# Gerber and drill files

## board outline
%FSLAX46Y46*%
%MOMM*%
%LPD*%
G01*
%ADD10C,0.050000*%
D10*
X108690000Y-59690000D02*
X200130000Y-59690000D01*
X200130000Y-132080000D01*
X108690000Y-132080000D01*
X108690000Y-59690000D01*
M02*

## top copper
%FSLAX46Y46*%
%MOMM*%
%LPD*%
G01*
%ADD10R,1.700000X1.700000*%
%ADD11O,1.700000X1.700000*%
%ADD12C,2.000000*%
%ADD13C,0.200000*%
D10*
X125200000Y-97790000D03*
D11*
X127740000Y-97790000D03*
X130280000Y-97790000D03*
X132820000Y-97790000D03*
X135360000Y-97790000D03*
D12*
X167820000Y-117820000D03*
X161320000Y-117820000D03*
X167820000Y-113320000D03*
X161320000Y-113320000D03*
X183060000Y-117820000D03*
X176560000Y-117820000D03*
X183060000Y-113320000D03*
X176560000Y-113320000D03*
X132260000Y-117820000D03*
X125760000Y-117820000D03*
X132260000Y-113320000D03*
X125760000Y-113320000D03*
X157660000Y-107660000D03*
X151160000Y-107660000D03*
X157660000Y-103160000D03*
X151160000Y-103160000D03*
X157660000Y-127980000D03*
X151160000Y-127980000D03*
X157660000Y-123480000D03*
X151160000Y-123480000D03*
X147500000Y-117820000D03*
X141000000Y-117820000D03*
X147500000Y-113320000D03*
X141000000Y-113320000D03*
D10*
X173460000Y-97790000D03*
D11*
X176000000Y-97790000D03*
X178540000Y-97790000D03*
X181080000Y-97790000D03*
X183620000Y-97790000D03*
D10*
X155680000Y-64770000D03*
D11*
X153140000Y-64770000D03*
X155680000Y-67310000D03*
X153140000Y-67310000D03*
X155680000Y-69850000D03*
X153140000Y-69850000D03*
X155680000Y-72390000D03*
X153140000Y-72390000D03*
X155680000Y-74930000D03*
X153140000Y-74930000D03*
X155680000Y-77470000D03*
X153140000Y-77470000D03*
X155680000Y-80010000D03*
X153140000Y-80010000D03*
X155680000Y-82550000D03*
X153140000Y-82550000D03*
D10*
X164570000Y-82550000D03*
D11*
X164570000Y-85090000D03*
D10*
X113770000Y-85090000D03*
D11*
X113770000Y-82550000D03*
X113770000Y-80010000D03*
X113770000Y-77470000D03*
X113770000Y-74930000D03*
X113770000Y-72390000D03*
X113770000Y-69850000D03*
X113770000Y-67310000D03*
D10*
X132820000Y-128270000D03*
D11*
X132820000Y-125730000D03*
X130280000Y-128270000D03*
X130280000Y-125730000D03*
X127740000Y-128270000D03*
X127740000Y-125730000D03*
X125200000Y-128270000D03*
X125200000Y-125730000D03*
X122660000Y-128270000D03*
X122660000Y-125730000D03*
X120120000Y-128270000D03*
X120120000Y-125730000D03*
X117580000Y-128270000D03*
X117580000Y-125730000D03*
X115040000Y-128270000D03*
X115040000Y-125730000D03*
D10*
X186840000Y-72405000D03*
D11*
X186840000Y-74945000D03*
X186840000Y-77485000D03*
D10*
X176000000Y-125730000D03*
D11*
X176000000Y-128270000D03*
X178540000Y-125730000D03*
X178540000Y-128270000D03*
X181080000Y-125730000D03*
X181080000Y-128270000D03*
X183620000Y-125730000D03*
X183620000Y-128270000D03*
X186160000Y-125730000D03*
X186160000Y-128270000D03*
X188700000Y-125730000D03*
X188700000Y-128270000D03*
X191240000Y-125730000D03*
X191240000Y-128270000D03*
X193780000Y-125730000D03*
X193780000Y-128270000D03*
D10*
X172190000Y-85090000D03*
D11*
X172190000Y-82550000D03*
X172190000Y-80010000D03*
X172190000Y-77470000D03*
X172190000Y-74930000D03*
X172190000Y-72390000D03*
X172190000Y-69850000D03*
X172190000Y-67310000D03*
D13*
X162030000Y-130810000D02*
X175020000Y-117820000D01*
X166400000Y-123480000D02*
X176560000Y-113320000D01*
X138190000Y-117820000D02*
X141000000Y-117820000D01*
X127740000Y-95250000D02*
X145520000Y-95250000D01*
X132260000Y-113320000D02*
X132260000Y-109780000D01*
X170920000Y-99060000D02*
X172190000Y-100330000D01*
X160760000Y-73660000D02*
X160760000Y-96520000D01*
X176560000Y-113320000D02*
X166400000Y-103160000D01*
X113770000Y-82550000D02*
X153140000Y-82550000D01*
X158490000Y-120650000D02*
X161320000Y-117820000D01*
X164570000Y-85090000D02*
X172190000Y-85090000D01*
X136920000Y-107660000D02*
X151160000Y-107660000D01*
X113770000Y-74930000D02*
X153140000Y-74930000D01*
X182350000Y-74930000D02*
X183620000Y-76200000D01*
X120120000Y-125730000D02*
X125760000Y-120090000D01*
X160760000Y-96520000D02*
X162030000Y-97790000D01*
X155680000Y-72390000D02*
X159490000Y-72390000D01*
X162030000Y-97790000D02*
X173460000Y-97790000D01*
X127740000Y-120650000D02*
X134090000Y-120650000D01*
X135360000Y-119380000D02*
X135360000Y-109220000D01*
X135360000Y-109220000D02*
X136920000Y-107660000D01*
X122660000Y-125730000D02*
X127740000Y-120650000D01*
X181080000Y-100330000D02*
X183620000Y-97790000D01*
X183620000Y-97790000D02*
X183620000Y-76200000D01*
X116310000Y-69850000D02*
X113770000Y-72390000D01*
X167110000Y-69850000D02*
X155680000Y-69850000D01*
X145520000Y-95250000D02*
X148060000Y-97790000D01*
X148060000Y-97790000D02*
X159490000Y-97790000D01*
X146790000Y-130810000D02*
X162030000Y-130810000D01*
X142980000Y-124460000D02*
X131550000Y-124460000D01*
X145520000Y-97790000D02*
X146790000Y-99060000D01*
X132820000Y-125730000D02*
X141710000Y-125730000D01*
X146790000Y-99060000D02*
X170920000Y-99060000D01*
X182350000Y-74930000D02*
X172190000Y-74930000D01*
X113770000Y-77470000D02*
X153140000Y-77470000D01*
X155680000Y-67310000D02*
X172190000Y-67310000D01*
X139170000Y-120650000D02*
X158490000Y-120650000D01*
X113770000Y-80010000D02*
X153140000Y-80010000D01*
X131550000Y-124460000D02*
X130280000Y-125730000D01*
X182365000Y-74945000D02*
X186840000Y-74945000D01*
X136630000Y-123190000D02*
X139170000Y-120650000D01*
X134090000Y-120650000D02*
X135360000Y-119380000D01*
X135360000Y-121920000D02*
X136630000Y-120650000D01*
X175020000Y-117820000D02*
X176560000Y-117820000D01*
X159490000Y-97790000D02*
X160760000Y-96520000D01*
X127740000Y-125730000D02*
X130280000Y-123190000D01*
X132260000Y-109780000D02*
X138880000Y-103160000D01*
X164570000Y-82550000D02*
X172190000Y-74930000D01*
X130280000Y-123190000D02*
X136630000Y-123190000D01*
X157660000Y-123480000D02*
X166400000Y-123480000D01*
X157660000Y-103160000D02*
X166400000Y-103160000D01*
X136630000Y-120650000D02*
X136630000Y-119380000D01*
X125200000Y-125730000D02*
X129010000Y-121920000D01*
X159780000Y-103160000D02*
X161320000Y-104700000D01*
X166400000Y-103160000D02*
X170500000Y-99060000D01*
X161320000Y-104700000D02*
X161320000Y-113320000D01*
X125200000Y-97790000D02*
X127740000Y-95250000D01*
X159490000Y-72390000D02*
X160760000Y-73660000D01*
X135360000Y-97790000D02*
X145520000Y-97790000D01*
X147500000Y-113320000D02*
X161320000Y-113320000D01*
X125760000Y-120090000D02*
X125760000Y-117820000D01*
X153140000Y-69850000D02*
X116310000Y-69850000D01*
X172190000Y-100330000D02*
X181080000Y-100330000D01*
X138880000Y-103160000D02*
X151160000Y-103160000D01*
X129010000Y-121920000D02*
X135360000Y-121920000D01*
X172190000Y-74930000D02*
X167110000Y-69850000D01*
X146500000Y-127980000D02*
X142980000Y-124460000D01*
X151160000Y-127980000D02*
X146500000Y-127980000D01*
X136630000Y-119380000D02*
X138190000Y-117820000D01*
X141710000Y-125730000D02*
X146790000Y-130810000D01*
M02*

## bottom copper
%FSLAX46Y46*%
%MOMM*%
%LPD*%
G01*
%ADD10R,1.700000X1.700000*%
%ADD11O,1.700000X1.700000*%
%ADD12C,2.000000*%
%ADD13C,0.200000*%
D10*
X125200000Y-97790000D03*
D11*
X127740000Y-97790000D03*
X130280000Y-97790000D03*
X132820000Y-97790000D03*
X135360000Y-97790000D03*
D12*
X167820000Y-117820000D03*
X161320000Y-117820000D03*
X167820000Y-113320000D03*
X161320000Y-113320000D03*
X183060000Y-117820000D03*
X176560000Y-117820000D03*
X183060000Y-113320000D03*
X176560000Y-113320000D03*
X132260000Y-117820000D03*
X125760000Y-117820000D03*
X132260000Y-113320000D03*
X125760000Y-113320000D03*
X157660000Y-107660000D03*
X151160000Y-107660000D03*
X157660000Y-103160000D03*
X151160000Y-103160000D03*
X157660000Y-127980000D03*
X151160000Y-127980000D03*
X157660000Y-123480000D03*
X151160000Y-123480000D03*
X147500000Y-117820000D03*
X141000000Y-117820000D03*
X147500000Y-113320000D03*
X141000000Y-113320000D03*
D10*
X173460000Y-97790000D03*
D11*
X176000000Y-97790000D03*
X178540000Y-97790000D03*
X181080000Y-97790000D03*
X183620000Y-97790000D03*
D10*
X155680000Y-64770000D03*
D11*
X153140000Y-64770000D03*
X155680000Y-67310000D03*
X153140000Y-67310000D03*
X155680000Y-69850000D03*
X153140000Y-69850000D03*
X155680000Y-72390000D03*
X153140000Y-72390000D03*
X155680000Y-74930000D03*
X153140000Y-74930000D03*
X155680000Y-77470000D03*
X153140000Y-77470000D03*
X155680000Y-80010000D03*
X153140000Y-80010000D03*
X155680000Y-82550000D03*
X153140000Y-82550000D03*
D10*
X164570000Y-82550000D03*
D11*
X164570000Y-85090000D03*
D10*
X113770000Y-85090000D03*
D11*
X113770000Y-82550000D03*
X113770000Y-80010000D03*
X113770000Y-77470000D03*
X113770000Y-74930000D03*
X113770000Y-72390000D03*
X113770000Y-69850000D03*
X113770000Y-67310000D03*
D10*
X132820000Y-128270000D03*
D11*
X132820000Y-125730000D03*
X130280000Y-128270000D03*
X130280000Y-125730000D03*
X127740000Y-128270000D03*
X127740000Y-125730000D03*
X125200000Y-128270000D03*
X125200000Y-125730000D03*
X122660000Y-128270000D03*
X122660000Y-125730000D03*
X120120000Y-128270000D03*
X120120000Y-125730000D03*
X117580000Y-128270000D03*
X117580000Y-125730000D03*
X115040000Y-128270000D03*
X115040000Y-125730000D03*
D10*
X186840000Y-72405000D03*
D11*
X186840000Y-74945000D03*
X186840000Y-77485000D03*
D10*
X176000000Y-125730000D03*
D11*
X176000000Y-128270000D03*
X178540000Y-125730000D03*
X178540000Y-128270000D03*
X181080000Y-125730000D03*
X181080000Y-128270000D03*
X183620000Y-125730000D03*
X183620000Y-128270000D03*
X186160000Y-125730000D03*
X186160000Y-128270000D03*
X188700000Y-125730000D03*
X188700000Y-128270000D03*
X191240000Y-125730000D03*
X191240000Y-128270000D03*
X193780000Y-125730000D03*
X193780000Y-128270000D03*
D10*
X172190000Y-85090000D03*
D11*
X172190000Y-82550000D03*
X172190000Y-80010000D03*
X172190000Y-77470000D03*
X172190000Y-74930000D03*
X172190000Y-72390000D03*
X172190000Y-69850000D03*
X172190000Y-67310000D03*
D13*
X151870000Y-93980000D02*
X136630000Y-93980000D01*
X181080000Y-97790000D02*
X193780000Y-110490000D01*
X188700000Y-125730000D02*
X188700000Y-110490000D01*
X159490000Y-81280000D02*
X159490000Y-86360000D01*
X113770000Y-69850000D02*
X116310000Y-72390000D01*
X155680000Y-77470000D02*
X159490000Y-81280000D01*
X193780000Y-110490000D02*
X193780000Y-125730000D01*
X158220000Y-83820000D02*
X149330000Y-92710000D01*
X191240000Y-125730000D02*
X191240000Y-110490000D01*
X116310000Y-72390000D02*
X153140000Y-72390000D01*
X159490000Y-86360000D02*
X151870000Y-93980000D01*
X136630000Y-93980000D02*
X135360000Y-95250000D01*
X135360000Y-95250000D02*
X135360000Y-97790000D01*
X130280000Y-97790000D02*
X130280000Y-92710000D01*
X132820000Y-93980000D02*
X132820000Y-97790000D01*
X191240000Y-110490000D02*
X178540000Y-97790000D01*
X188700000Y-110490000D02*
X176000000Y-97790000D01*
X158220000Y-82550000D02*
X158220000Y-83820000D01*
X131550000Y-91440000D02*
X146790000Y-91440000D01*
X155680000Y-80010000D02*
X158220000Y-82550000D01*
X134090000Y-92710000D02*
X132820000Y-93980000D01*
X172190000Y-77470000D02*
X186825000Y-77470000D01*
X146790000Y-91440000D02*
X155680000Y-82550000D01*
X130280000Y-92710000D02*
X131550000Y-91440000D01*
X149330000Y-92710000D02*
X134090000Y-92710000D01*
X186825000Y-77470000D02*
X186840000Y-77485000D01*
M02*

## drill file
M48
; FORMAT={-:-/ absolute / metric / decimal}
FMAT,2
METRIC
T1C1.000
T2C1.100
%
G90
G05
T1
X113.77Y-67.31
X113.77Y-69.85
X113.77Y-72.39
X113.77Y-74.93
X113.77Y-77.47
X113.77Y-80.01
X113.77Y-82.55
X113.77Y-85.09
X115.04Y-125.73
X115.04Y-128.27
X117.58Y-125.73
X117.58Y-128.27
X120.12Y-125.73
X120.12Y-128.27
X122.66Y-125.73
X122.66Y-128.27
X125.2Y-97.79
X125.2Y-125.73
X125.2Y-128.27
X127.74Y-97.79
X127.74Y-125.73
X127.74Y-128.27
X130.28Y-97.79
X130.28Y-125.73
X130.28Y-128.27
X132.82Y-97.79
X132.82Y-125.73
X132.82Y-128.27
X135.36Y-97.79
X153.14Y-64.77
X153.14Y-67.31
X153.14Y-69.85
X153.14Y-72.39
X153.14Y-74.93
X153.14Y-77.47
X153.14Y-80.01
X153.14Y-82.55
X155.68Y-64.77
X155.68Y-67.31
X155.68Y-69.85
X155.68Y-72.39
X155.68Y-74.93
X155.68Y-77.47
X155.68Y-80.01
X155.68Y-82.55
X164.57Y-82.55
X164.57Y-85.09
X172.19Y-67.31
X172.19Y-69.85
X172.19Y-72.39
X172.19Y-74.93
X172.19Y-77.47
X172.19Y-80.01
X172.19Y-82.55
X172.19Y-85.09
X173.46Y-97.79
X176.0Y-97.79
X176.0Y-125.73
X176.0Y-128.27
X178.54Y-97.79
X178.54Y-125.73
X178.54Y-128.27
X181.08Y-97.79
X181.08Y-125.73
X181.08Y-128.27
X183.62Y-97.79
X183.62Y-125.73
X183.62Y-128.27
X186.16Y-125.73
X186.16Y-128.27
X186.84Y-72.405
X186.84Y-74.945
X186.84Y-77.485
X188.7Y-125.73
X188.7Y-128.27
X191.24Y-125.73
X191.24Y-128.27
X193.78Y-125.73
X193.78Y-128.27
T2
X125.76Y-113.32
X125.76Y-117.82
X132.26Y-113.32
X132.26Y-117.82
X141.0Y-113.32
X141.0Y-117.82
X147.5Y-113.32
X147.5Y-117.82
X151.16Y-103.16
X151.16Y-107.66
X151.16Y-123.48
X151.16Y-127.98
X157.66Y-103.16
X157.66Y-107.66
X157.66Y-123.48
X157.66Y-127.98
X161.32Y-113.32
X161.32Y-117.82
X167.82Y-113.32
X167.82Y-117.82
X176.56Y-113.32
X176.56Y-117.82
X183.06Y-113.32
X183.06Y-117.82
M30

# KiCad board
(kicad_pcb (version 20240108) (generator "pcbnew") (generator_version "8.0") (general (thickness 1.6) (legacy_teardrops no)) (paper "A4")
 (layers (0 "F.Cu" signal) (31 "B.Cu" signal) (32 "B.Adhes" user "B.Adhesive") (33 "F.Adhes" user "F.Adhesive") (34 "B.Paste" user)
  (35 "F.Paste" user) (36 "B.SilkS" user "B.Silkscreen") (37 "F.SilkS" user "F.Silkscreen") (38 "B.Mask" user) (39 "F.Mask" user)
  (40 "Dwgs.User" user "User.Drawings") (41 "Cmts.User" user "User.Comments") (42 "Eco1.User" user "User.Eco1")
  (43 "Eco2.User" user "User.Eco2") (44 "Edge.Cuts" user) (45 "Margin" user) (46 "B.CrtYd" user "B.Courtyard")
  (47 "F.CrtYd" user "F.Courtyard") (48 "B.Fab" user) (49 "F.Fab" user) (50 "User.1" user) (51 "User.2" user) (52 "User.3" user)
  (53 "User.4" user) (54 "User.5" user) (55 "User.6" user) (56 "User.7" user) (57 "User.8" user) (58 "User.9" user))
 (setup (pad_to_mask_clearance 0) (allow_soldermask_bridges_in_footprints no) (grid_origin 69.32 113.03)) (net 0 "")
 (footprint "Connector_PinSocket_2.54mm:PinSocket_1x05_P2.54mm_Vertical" (layer "F.Cu") (at 125.2 97.79 90)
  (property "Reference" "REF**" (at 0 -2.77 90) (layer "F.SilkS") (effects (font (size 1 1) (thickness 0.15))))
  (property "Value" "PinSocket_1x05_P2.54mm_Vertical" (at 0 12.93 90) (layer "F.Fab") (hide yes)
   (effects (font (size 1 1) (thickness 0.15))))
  (pad "1" thru_hole rect (at 0 0 90) (size 1.7 1.7) (drill 1) (layers "*.Cu" "*.Mask") (remove_unused_layers no))
  (pad "2" thru_hole oval (at 0 2.54 90) (size 1.7 1.7) (drill 1) (layers "*.Cu" "*.Mask") (remove_unused_layers no))
  (pad "3" thru_hole oval (at 0 5.08 90) (size 1.7 1.7) (drill 1) (layers "*.Cu" "*.Mask") (remove_unused_layers no))
  (pad "4" thru_hole oval (at 0 7.62 90) (size 1.7 1.7) (drill 1) (layers "*.Cu" "*.Mask") (remove_unused_layers no))
  (pad "5" thru_hole oval (at 0 10.16 90) (size 1.7 1.7) (drill 1) (layers "*.Cu" "*.Mask") (remove_unused_layers no)))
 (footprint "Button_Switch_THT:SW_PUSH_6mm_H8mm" (layer "F.Cu") (at 167.82 117.82 180)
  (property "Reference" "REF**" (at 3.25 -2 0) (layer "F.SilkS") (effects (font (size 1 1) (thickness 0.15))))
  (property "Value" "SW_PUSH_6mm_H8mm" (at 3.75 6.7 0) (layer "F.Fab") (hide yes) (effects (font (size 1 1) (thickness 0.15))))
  (pad "1" thru_hole circle (at 0 0 270) (size 2 2) (drill 1.1) (layers "*.Cu" "*.Mask") (remove_unused_layers no))
  (pad "1" thru_hole circle (at 6.5 0 270) (size 2 2) (drill 1.1) (layers "*.Cu" "*.Mask") (remove_unused_layers no))
  (pad "2" thru_hole circle (at 0 4.5 270) (size 2 2) (drill 1.1) (layers "*.Cu" "*.Mask") (remove_unused_layers no))
  (pad "2" thru_hole circle (at 6.5 4.5 270) (size 2 2) (drill 1.1) (layers "*.Cu" "*.Mask") (remove_unused_layers no)))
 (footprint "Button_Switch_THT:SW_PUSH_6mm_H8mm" (layer "F.Cu") (at 183.06 117.82 180)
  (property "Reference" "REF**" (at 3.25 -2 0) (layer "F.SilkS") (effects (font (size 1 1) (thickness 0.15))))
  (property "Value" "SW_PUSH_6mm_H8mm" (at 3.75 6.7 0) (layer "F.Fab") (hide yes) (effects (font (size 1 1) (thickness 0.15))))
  (pad "1" thru_hole circle (at 0 0 270) (size 2 2) (drill 1.1) (layers "*.Cu" "*.Mask") (remove_unused_layers no))
  (pad "1" thru_hole circle (at 6.5 0 270) (size 2 2) (drill 1.1) (layers "*.Cu" "*.Mask") (remove_unused_layers no))
  (pad "2" thru_hole circle (at 0 4.5 270) (size 2 2) (drill 1.1) (layers "*.Cu" "*.Mask") (remove_unused_layers no))
  (pad "2" thru_hole circle (at 6.5 4.5 270) (size 2 2) (drill 1.1) (layers "*.Cu" "*.Mask") (remove_unused_layers no)))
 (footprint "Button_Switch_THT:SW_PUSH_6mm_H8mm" (layer "F.Cu") (at 132.26 117.82 180)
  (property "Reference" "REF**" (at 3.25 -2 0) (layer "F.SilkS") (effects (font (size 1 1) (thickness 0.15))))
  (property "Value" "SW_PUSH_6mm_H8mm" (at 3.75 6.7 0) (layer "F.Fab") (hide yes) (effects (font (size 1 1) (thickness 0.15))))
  (pad "1" thru_hole circle (at 0 0 270) (size 2 2) (drill 1.1) (layers "*.Cu" "*.Mask") (remove_unused_layers no))
  (pad "1" thru_hole circle (at 6.5 0 270) (size 2 2) (drill 1.1) (layers "*.Cu" "*.Mask") (remove_unused_layers no))
  (pad "2" thru_hole circle (at 0 4.5 270) (size 2 2) (drill 1.1) (layers "*.Cu" "*.Mask") (remove_unused_layers no))
  (pad "2" thru_hole circle (at 6.5 4.5 270) (size 2 2) (drill 1.1) (layers "*.Cu" "*.Mask") (remove_unused_layers no)))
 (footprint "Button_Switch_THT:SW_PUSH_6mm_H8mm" (layer "F.Cu") (at 157.66 107.66 180)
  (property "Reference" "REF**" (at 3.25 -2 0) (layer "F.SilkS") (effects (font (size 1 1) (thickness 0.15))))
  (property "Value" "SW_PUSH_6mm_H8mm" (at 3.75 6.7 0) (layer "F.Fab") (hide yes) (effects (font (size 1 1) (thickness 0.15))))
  (pad "1" thru_hole circle (at 0 0 270) (size 2 2) (drill 1.1) (layers "*.Cu" "*.Mask") (remove_unused_layers no))
  (pad "1" thru_hole circle (at 6.5 0 270) (size 2 2) (drill 1.1) (layers "*.Cu" "*.Mask") (remove_unused_layers no))
  (pad "2" thru_hole circle (at 0 4.5 270) (size 2 2) (drill 1.1) (layers "*.Cu" "*.Mask") (remove_unused_layers no))
  (pad "2" thru_hole circle (at 6.5 4.5 270) (size 2 2) (drill 1.1) (layers "*.Cu" "*.Mask") (remove_unused_layers no)))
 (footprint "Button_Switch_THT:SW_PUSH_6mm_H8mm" (layer "F.Cu") (at 157.66 127.98 180)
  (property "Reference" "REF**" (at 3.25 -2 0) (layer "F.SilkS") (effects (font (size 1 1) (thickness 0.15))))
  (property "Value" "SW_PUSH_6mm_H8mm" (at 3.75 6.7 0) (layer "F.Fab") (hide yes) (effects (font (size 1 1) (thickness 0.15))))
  (pad "1" thru_hole circle (at 0 0 270) (size 2 2) (drill 1.1) (layers "*.Cu" "*.Mask") (remove_unused_layers no))
  (pad "1" thru_hole circle (at 6.5 0 270) (size 2 2) (drill 1.1) (layers "*.Cu" "*.Mask") (remove_unused_layers no))
  (pad "2" thru_hole circle (at 0 4.5 270) (size 2 2) (drill 1.1) (layers "*.Cu" "*.Mask") (remove_unused_layers no))
  (pad "2" thru_hole circle (at 6.5 4.5 270) (size 2 2) (drill 1.1) (layers "*.Cu" "*.Mask") (remove_unused_layers no)))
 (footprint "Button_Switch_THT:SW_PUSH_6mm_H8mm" (layer "F.Cu") (at 147.5 117.82 180)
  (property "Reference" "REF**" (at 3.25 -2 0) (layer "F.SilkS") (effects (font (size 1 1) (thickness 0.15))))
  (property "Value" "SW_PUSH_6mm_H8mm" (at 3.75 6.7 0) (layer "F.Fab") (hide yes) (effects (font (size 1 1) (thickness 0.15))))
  (pad "1" thru_hole circle (at 0 0 270) (size 2 2) (drill 1.1) (layers "*.Cu" "*.Mask") (remove_unused_layers no))
  (pad "1" thru_hole circle (at 6.5 0 270) (size 2 2) (drill 1.1) (layers "*.Cu" "*.Mask") (remove_unused_layers no))
  (pad "2" thru_hole circle (at 0 4.5 270) (size 2 2) (drill 1.1) (layers "*.Cu" "*.Mask") (remove_unused_layers no))
  (pad "2" thru_hole circle (at 6.5 4.5 270) (size 2 2) (drill 1.1) (layers "*.Cu" "*.Mask") (remove_unused_layers no)))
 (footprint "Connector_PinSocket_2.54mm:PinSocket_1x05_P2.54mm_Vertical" (layer "F.Cu") (at 173.46 97.79 90)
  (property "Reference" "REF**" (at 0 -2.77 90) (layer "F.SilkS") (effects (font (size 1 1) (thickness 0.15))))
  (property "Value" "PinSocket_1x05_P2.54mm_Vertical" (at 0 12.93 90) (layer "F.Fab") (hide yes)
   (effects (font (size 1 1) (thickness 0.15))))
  (pad "1" thru_hole rect (at 0 0 90) (size 1.7 1.7) (drill 1) (layers "*.Cu" "*.Mask") (remove_unused_layers no))
  (pad "2" thru_hole oval (at 0 2.54 90) (size 1.7 1.7) (drill 1) (layers "*.Cu" "*.Mask") (remove_unused_layers no))
  (pad "3" thru_hole oval (at 0 5.08 90) (size 1.7 1.7) (drill 1) (layers "*.Cu" "*.Mask") (remove_unused_layers no))
  (pad "4" thru_hole oval (at 0 7.62 90) (size 1.7 1.7) (drill 1) (layers "*.Cu" "*.Mask") (remove_unused_layers no))
  (pad "5" thru_hole oval (at 0 10.16 90) (size 1.7 1.7) (drill 1) (layers "*.Cu" "*.Mask") (remove_unused_layers no)))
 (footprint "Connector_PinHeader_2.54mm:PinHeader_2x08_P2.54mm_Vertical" (layer "B.Cu") (at 155.68 64.77 180)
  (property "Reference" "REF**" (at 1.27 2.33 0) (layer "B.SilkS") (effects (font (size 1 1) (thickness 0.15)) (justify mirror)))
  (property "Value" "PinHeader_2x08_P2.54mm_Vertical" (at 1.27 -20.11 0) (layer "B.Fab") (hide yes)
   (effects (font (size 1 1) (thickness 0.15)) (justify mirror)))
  (pad "1" thru_hole rect (at 0 0 180) (size 1.7 1.7) (drill 1) (layers "*.Cu" "*.Mask") (remove_unused_layers no))
  (pad "2" thru_hole oval (at 2.54 0 180) (size 1.7 1.7) (drill 1) (layers "*.Cu" "*.Mask") (remove_unused_layers no))
  (pad "3" thru_hole oval (at 0 -2.54 180) (size 1.7 1.7) (drill 1) (layers "*.Cu" "*.Mask") (remove_unused_layers no))
  (pad "4" thru_hole oval (at 2.54 -2.54 180) (size 1.7 1.7) (drill 1) (layers "*.Cu" "*.Mask") (remove_unused_layers no))
  (pad "5" thru_hole oval (at 0 -5.08 180) (size 1.7 1.7) (drill 1) (layers "*.Cu" "*.Mask") (remove_unused_layers no))
  (pad "6" thru_hole oval (at 2.54 -5.08 180) (size 1.7 1.7) (drill 1) (layers "*.Cu" "*.Mask") (remove_unused_layers no))
  (pad "7" thru_hole oval (at 0 -7.62 180) (size 1.7 1.7) (drill 1) (layers "*.Cu" "*.Mask") (remove_unused_layers no))
  (pad "8" thru_hole oval (at 2.54 -7.62 180) (size 1.7 1.7) (drill 1) (layers "*.Cu" "*.Mask") (remove_unused_layers no))
  (pad "9" thru_hole oval (at 0 -10.16 180) (size 1.7 1.7) (drill 1) (layers "*.Cu" "*.Mask") (remove_unused_layers no))
  (pad "10" thru_hole oval (at 2.54 -10.16 180) (size 1.7 1.7) (drill 1) (layers "*.Cu" "*.Mask") (remove_unused_layers no))
  (pad "11" thru_hole oval (at 0 -12.7 180) (size 1.7 1.7) (drill 1) (layers "*.Cu" "*.Mask") (remove_unused_layers no))
  (pad "12" thru_hole oval (at 2.54 -12.7 180) (size 1.7 1.7) (drill 1) (layers "*.Cu" "*.Mask") (remove_unused_layers no))
  (pad "13" thru_hole oval (at 0 -15.24 180) (size 1.7 1.7) (drill 1) (layers "*.Cu" "*.Mask") (remove_unused_layers no))
  (pad "14" thru_hole oval (at 2.54 -15.24 180) (size 1.7 1.7) (drill 1) (layers "*.Cu" "*.Mask") (remove_unused_layers no))
  (pad "15" thru_hole oval (at 0 -17.78 180) (size 1.7 1.7) (drill 1) (layers "*.Cu" "*.Mask") (remove_unused_layers no))
  (pad "16" thru_hole oval (at 2.54 -17.78 180) (size 1.7 1.7) (drill 1) (layers "*.Cu" "*.Mask") (remove_unused_layers no)))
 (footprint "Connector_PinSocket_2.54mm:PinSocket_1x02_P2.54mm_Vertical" (layer "B.Cu") (at 164.57 82.55 180)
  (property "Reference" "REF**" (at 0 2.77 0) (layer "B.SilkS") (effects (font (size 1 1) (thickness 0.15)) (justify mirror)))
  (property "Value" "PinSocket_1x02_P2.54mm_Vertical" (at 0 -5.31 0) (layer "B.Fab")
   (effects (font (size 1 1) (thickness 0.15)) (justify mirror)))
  (pad "1" thru_hole rect (at 0 0 180) (size 1.7 1.7) (drill 1) (layers "*.Cu" "*.Mask") (remove_unused_layers no))
  (pad "2" thru_hole oval (at 0 -2.54 180) (size 1.7 1.7) (drill 1) (layers "*.Cu" "*.Mask") (remove_unused_layers no)))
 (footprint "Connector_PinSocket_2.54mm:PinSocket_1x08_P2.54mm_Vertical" (layer "B.Cu") (at 113.77 85.09)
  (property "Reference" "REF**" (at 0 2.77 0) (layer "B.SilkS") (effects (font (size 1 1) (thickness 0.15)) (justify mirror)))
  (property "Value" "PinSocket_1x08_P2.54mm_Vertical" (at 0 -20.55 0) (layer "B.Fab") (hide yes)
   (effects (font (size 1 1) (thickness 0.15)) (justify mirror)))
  (pad "1" thru_hole rect (at 0 0) (size 1.7 1.7) (drill 1) (layers "*.Cu" "*.Mask") (remove_unused_layers no))
  (pad "2" thru_hole oval (at 0 -2.54) (size 1.7 1.7) (drill 1) (layers "*.Cu" "*.Mask") (remove_unused_layers no))
  (pad "3" thru_hole oval (at 0 -5.08) (size 1.7 1.7) (drill 1) (layers "*.Cu" "*.Mask") (remove_unused_layers no))
  (pad "4" thru_hole oval (at 0 -7.62) (size 1.7 1.7) (drill 1) (layers "*.Cu" "*.Mask") (remove_unused_layers no))
  (pad "5" thru_hole oval (at 0 -10.16) (size 1.7 1.7) (drill 1) (layers "*.Cu" "*.Mask") (remove_unused_layers no))
  (pad "6" thru_hole oval (at 0 -12.7) (size 1.7 1.7) (drill 1) (layers "*.Cu" "*.Mask") (remove_unused_layers no))
  (pad "7" thru_hole oval (at 0 -15.24) (size 1.7 1.7) (drill 1) (layers "*.Cu" "*.Mask") (remove_unused_layers no))
  (pad "8" thru_hole oval (at 0 -17.78) (size 1.7 1.7) (drill 1) (layers "*.Cu" "*.Mask") (remove_unused_layers no)))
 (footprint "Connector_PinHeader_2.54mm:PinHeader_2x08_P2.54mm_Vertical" (layer "B.Cu") (at 132.82 128.27 90)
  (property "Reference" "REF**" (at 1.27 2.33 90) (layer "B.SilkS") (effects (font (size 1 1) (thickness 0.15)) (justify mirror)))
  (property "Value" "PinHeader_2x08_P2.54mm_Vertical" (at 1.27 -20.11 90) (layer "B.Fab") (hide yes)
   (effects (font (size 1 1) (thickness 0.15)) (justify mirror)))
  (pad "1" thru_hole rect (at 0 0 90) (size 1.7 1.7) (drill 1) (layers "*.Cu" "*.Mask") (remove_unused_layers no))
  (pad "2" thru_hole oval (at 2.54 0 90) (size 1.7 1.7) (drill 1) (layers "*.Cu" "*.Mask") (remove_unused_layers no))
  (pad "3" thru_hole oval (at 0 -2.54 90) (size 1.7 1.7) (drill 1) (layers "*.Cu" "*.Mask") (remove_unused_layers no))
  (pad "4" thru_hole oval (at 2.54 -2.54 90) (size 1.7 1.7) (drill 1) (layers "*.Cu" "*.Mask") (remove_unused_layers no))
  (pad "5" thru_hole oval (at 0 -5.08 90) (size 1.7 1.7) (drill 1) (layers "*.Cu" "*.Mask") (remove_unused_layers no))
  (pad "6" thru_hole oval (at 2.54 -5.08 90) (size 1.7 1.7) (drill 1) (layers "*.Cu" "*.Mask") (remove_unused_layers no))
  (pad "7" thru_hole oval (at 0 -7.62 90) (size 1.7 1.7) (drill 1) (layers "*.Cu" "*.Mask") (remove_unused_layers no))
  (pad "8" thru_hole oval (at 2.54 -7.62 90) (size 1.7 1.7) (drill 1) (layers "*.Cu" "*.Mask") (remove_unused_layers no))
  (pad "9" thru_hole oval (at 0 -10.16 90) (size 1.7 1.7) (drill 1) (layers "*.Cu" "*.Mask") (remove_unused_layers no))
  (pad "10" thru_hole oval (at 2.54 -10.16 90) (size 1.7 1.7) (drill 1) (layers "*.Cu" "*.Mask") (remove_unused_layers no))
  (pad "11" thru_hole oval (at 0 -12.7 90) (size 1.7 1.7) (drill 1) (layers "*.Cu" "*.Mask") (remove_unused_layers no))
  (pad "12" thru_hole oval (at 2.54 -12.7 90) (size 1.7 1.7) (drill 1) (layers "*.Cu" "*.Mask") (remove_unused_layers no))
  (pad "13" thru_hole oval (at 0 -15.24 90) (size 1.7 1.7) (drill 1) (layers "*.Cu" "*.Mask") (remove_unused_layers no))
  (pad "14" thru_hole oval (at 2.54 -15.24 90) (size 1.7 1.7) (drill 1) (layers "*.Cu" "*.Mask") (remove_unused_layers no))
  (pad "15" thru_hole oval (at 0 -17.78 90) (size 1.7 1.7) (drill 1) (layers "*.Cu" "*.Mask") (remove_unused_layers no))
  (pad "16" thru_hole oval (at 2.54 -17.78 90) (size 1.7 1.7) (drill 1) (layers "*.Cu" "*.Mask") (remove_unused_layers no)))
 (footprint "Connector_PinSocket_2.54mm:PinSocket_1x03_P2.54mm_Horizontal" (layer "B.Cu") (at 186.84 72.405 180)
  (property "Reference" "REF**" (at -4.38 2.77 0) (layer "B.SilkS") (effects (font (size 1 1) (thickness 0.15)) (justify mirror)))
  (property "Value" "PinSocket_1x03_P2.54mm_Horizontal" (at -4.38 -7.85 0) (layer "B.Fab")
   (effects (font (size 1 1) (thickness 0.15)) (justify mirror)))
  (pad "1" thru_hole rect (at 0 0 180) (size 1.7 1.7) (drill 1) (layers "*.Cu" "*.Mask") (remove_unused_layers no))
  (pad "2" thru_hole oval (at 0 -2.54 180) (size 1.7 1.7) (drill 1) (layers "*.Cu" "*.Mask") (remove_unused_layers no))
  (pad "3" thru_hole oval (at 0 -5.08 180) (size 1.7 1.7) (drill 1) (layers "*.Cu" "*.Mask") (remove_unused_layers no)))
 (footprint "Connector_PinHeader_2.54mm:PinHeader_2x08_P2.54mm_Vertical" (layer "B.Cu") (at 176 125.73 -90)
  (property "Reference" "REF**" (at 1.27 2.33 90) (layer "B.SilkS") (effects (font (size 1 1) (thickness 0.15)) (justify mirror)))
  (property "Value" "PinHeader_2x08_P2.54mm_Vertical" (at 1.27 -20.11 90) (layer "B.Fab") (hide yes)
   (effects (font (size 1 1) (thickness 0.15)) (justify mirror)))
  (pad "1" thru_hole rect (at 0 0 270) (size 1.7 1.7) (drill 1) (layers "*.Cu" "*.Mask") (remove_unused_layers no))
  (pad "2" thru_hole oval (at 2.54 0 270) (size 1.7 1.7) (drill 1) (layers "*.Cu" "*.Mask") (remove_unused_layers no))
  (pad "3" thru_hole oval (at 0 -2.54 270) (size 1.7 1.7) (drill 1) (layers "*.Cu" "*.Mask") (remove_unused_layers no))
  (pad "4" thru_hole oval (at 2.54 -2.54 270) (size 1.7 1.7) (drill 1) (layers "*.Cu" "*.Mask") (remove_unused_layers no))
  (pad "5" thru_hole oval (at 0 -5.08 270) (size 1.7 1.7) (drill 1) (layers "*.Cu" "*.Mask") (remove_unused_layers no))
  (pad "6" thru_hole oval (at 2.54 -5.08 270) (size 1.7 1.7) (drill 1) (layers "*.Cu" "*.Mask") (remove_unused_layers no))
  (pad "7" thru_hole oval (at 0 -7.62 270) (size 1.7 1.7) (drill 1) (layers "*.Cu" "*.Mask") (remove_unused_layers no))
  (pad "8" thru_hole oval (at 2.54 -7.62 270) (size 1.7 1.7) (drill 1) (layers "*.Cu" "*.Mask") (remove_unused_layers no))
  (pad "9" thru_hole oval (at 0 -10.16 270) (size 1.7 1.7) (drill 1) (layers "*.Cu" "*.Mask") (remove_unused_layers no))
  (pad "10" thru_hole oval (at 2.54 -10.16 270) (size 1.7 1.7) (drill 1) (layers "*.Cu" "*.Mask") (remove_unused_layers no))
  (pad "11" thru_hole oval (at 0 -12.7 270) (size 1.7 1.7) (drill 1) (layers "*.Cu" "*.Mask") (remove_unused_layers no))
  (pad "12" thru_hole oval (at 2.54 -12.7 270) (size 1.7 1.7) (drill 1) (layers "*.Cu" "*.Mask") (remove_unused_layers no))
  (pad "13" thru_hole oval (at 0 -15.24 270) (size 1.7 1.7) (drill 1) (layers "*.Cu" "*.Mask") (remove_unused_layers no))
  (pad "14" thru_hole oval (at 2.54 -15.24 270) (size 1.7 1.7) (drill 1) (layers "*.Cu" "*.Mask") (remove_unused_layers no))
  (pad "15" thru_hole oval (at 0 -17.78 270) (size 1.7 1.7) (drill 1) (layers "*.Cu" "*.Mask") (remove_unused_layers no))
  (pad "16" thru_hole oval (at 2.54 -17.78 270) (size 1.7 1.7) (drill 1) (layers "*.Cu" "*.Mask") (remove_unused_layers no)))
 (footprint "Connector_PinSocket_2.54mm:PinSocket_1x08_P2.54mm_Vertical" (layer "B.Cu") (at 172.19 85.09)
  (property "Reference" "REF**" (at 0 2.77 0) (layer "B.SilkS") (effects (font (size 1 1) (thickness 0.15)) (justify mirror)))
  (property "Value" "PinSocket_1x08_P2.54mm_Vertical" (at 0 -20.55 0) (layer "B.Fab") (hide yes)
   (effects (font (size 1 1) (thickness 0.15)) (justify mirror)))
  (pad "1" thru_hole rect (at 0 0) (size 1.7 1.7) (drill 1) (layers "*.Cu" "*.Mask") (remove_unused_layers no))
  (pad "2" thru_hole oval (at 0 -2.54) (size 1.7 1.7) (drill 1) (layers "*.Cu" "*.Mask") (remove_unused_layers no))
  (pad "3" thru_hole oval (at 0 -5.08) (size 1.7 1.7) (drill 1) (layers "*.Cu" "*.Mask") (remove_unused_layers no))
  (pad "4" thru_hole oval (at 0 -7.62) (size 1.7 1.7) (drill 1) (layers "*.Cu" "*.Mask") (remove_unused_layers no))
  (pad "5" thru_hole oval (at 0 -10.16) (size 1.7 1.7) (drill 1) (layers "*.Cu" "*.Mask") (remove_unused_layers no))
  (pad "6" thru_hole oval (at 0 -12.7) (size 1.7 1.7) (drill 1) (layers "*.Cu" "*.Mask") (remove_unused_layers no))
  (pad "7" thru_hole oval (at 0 -15.24) (size 1.7 1.7) (drill 1) (layers "*.Cu" "*.Mask") (remove_unused_layers no))
  (pad "8" thru_hole oval (at 0 -17.78) (size 1.7 1.7) (drill 1) (layers "*.Cu" "*.Mask") (remove_unused_layers no)))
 (gr_rect (start 108.69 59.69) (end 200.13 132.08) (stroke (width 0.05) (type default)) (fill none) (layer "Edge.Cuts"))
 (segment (start 162.03 130.81) (end 175.02 117.82) (width 0.2) (layer "F.Cu") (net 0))
 (segment (start 166.4 123.48) (end 176.56 113.32) (width 0.2) (layer "F.Cu") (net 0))
 (segment (start 138.19 117.82) (end 141 117.82) (width 0.2) (layer "F.Cu") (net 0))
 (segment (start 127.74 95.25) (end 145.52 95.25) (width 0.2) (layer "F.Cu") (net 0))
 (segment (start 132.26 113.32) (end 132.26 109.78) (width 0.2) (layer "F.Cu") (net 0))
 (segment (start 170.92 99.06) (end 172.19 100.33) (width 0.2) (layer "F.Cu") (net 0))
 (segment (start 160.76 73.66) (end 160.76 96.52) (width 0.2) (layer "F.Cu") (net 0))
 (segment (start 176.56 113.32) (end 166.4 103.16) (width 0.2) (layer "F.Cu") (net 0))
 (segment (start 113.77 82.55) (end 153.14 82.55) (width 0.2) (layer "F.Cu") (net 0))
 (segment (start 158.49 120.65) (end 161.32 117.82) (width 0.2) (layer "F.Cu") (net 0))
 (segment (start 164.57 85.09) (end 172.19 85.09) (width 0.2) (layer "F.Cu") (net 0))
 (segment (start 136.92 107.66) (end 151.16 107.66) (width 0.2) (layer "F.Cu") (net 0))
 (segment (start 113.77 74.93) (end 153.14 74.93) (width 0.2) (layer "F.Cu") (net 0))
 (segment (start 182.35 74.93) (end 183.62 76.2) (width 0.2) (layer "F.Cu") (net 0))
 (segment (start 120.12 125.73) (end 125.76 120.09) (width 0.2) (layer "F.Cu") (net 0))
 (segment (start 160.76 96.52) (end 162.03 97.79) (width 0.2) (layer "F.Cu") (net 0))
 (segment (start 155.68 72.39) (end 159.49 72.39) (width 0.2) (layer "F.Cu") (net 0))
 (segment (start 162.03 97.79) (end 173.46 97.79) (width 0.2) (layer "F.Cu") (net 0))
 (segment (start 127.74 120.65) (end 134.09 120.65) (width 0.2) (layer "F.Cu") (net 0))
 (segment (start 135.36 119.38) (end 135.36 109.22) (width 0.2) (layer "F.Cu") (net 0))
 (segment (start 135.36 109.22) (end 136.92 107.66) (width 0.2) (layer "F.Cu") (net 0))
 (segment (start 122.66 125.73) (end 127.74 120.65) (width 0.2) (layer "F.Cu") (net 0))
 (segment (start 181.08 100.33) (end 183.62 97.79) (width 0.2) (layer "F.Cu") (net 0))
 (segment (start 183.62 97.79) (end 183.62 76.2) (width 0.2) (layer "F.Cu") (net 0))
 (segment (start 116.31 69.85) (end 113.77 72.39) (width 0.2) (layer "F.Cu") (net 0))
 (segment (start 167.11 69.85) (end 155.68 69.85) (width 0.2) (layer "F.Cu") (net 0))
 (segment (start 145.52 95.25) (end 148.06 97.79) (width 0.2) (layer "F.Cu") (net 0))
 (segment (start 148.06 97.79) (end 159.49 97.79) (width 0.2) (layer "F.Cu") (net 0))
 (segment (start 146.79 130.81) (end 162.03 130.81) (width 0.2) (layer "F.Cu") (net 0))
 (segment (start 142.98 124.46) (end 131.55 124.46) (width 0.2) (layer "F.Cu") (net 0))
 (segment (start 145.52 97.79) (end 146.79 99.06) (width 0.2) (layer "F.Cu") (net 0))
 (segment (start 132.82 125.73) (end 141.71 125.73) (width 0.2) (layer "F.Cu") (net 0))
 (segment (start 146.79 99.06) (end 170.92 99.06) (width 0.2) (layer "F.Cu") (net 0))
 (segment (start 182.35 74.93) (end 172.19 74.93) (width 0.2) (layer "F.Cu") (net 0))
 (segment (start 113.77 77.47) (end 153.14 77.47) (width 0.2) (layer "F.Cu") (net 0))
 (segment (start 155.68 67.31) (end 172.19 67.31) (width 0.2) (layer "F.Cu") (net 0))
 (segment (start 139.17 120.65) (end 158.49 120.65) (width 0.2) (layer "F.Cu") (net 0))
 (segment (start 113.77 80.01) (end 153.14 80.01) (width 0.2) (layer "F.Cu") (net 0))
 (segment (start 131.55 124.46) (end 130.28 125.73) (width 0.2) (layer "F.Cu") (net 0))
 (segment (start 182.365 74.945) (end 186.84 74.945) (width 0.2) (layer "F.Cu") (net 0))
 (segment (start 136.63 123.19) (end 139.17 120.65) (width 0.2) (layer "F.Cu") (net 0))
 (segment (start 134.09 120.65) (end 135.36 119.38) (width 0.2) (layer "F.Cu") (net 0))
 (segment (start 135.36 121.92) (end 136.63 120.65) (width 0.2) (layer "F.Cu") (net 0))
 (segment (start 175.02 117.82) (end 176.56 117.82) (width 0.2) (layer "F.Cu") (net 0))
 (segment (start 159.49 97.79) (end 160.76 96.52) (width 0.2) (layer "F.Cu") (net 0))
 (segment (start 127.74 125.73) (end 130.28 123.19) (width 0.2) (layer "F.Cu") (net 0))
 (segment (start 132.26 109.78) (end 138.88 103.16) (width 0.2) (layer "F.Cu") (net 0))
 (segment (start 164.57 82.55) (end 172.19 74.93) (width 0.2) (layer "F.Cu") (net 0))
 (segment (start 130.28 123.19) (end 136.63 123.19) (width 0.2) (layer "F.Cu") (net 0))
 (segment (start 157.66 123.48) (end 166.4 123.48) (width 0.2) (layer "F.Cu") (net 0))
 (segment (start 157.66 103.16) (end 166.4 103.16) (width 0.2) (layer "F.Cu") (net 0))
 (segment (start 136.63 120.65) (end 136.63 119.38) (width 0.2) (layer "F.Cu") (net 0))
 (segment (start 125.2 125.73) (end 129.01 121.92) (width 0.2) (layer "F.Cu") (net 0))
 (segment (start 159.78 103.16) (end 161.32 104.7) (width 0.2) (layer "F.Cu") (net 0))
 (segment (start 166.4 103.16) (end 170.5 99.06) (width 0.2) (layer "F.Cu") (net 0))
 (segment (start 161.32 104.7) (end 161.32 113.32) (width 0.2) (layer "F.Cu") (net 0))
 (segment (start 125.2 97.79) (end 127.74 95.25) (width 0.2) (layer "F.Cu") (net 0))
 (segment (start 159.49 72.39) (end 160.76 73.66) (width 0.2) (layer "F.Cu") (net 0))
 (segment (start 135.36 97.79) (end 145.52 97.79) (width 0.2) (layer "F.Cu") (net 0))
 (segment (start 147.5 113.32) (end 161.32 113.32) (width 0.2) (layer "F.Cu") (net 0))
 (segment (start 125.76 120.09) (end 125.76 117.82) (width 0.2) (layer "F.Cu") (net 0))
 (segment (start 153.14 69.85) (end 116.31 69.85) (width 0.2) (layer "F.Cu") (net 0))
 (segment (start 172.19 100.33) (end 181.08 100.33) (width 0.2) (layer "F.Cu") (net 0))
 (segment (start 138.88 103.16) (end 151.16 103.16) (width 0.2) (layer "F.Cu") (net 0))
 (segment (start 129.01 121.92) (end 135.36 121.92) (width 0.2) (layer "F.Cu") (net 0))
 (segment (start 172.19 74.93) (end 167.11 69.85) (width 0.2) (layer "F.Cu") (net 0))
 (segment (start 146.5 127.98) (end 142.98 124.46) (width 0.2) (layer "F.Cu") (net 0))
 (segment (start 151.16 127.98) (end 146.5 127.98) (width 0.2) (layer "F.Cu") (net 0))
 (segment (start 136.63 119.38) (end 138.19 117.82) (width 0.2) (layer "F.Cu") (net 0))
 (segment (start 141.71 125.73) (end 146.79 130.81) (width 0.2) (layer "F.Cu") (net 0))
 (segment (start 151.87 93.98) (end 136.63 93.98) (width 0.2) (layer "B.Cu") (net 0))
 (segment (start 181.08 97.79) (end 193.78 110.49) (width 0.2) (layer "B.Cu") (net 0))
 (segment (start 188.7 125.73) (end 188.7 110.49) (width 0.2) (layer "B.Cu") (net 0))
 (segment (start 159.49 81.28) (end 159.49 86.36) (width 0.2) (layer "B.Cu") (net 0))
 (segment (start 113.77 69.85) (end 116.31 72.39) (width 0.2) (layer "B.Cu") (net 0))
 (segment (start 155.68 77.47) (end 159.49 81.28) (width 0.2) (layer "B.Cu") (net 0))
 (segment (start 193.78 110.49) (end 193.78 125.73) (width 0.2) (layer "B.Cu") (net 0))
 (segment (start 158.22 83.82) (end 149.33 92.71) (width 0.2) (layer "B.Cu") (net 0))
 (segment (start 191.24 125.73) (end 191.24 110.49) (width 0.2) (layer "B.Cu") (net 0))
 (segment (start 116.31 72.39) (end 153.14 72.39) (width 0.2) (layer "B.Cu") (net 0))
 (segment (start 159.49 86.36) (end 151.87 93.98) (width 0.2) (layer "B.Cu") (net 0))
 (segment (start 136.63 93.98) (end 135.36 95.25) (width 0.2) (layer "B.Cu") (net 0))
 (segment (start 135.36 95.25) (end 135.36 97.79) (width 0.2) (layer "B.Cu") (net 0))
 (segment (start 130.28 97.79) (end 130.28 92.71) (width 0.2) (layer "B.Cu") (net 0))
 (segment (start 132.82 93.98) (end 132.82 97.79) (width 0.2) (layer "B.Cu") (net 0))
 (segment (start 191.24 110.49) (end 178.54 97.79) (width 0.2) (layer "B.Cu") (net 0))
 (segment (start 188.7 110.49) (end 176 97.79) (width 0.2) (layer "B.Cu") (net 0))
 (segment (start 158.22 82.55) (end 158.22 83.82) (width 0.2) (layer "B.Cu") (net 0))
 (segment (start 131.55 91.44) (end 146.79 91.44) (width 0.2) (layer "B.Cu") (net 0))
 (segment (start 155.68 80.01) (end 158.22 82.55) (width 0.2) (layer "B.Cu") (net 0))
 (segment (start 134.09 92.71) (end 132.82 93.98) (width 0.2) (layer "B.Cu") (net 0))
 (segment (start 172.19 77.47) (end 186.825 77.47) (width 0.2) (layer "B.Cu") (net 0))
 (segment (start 146.79 91.44) (end 155.68 82.55) (width 0.2) (layer "B.Cu") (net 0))
 (segment (start 130.28 92.71) (end 131.55 91.44) (width 0.2) (layer "B.Cu") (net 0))
 (segment (start 149.33 92.71) (end 134.09 92.71) (width 0.2) (layer "B.Cu") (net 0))
 (segment (start 186.825 77.47) (end 186.84 77.485) (width 0.2) (layer "B.Cu") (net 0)))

